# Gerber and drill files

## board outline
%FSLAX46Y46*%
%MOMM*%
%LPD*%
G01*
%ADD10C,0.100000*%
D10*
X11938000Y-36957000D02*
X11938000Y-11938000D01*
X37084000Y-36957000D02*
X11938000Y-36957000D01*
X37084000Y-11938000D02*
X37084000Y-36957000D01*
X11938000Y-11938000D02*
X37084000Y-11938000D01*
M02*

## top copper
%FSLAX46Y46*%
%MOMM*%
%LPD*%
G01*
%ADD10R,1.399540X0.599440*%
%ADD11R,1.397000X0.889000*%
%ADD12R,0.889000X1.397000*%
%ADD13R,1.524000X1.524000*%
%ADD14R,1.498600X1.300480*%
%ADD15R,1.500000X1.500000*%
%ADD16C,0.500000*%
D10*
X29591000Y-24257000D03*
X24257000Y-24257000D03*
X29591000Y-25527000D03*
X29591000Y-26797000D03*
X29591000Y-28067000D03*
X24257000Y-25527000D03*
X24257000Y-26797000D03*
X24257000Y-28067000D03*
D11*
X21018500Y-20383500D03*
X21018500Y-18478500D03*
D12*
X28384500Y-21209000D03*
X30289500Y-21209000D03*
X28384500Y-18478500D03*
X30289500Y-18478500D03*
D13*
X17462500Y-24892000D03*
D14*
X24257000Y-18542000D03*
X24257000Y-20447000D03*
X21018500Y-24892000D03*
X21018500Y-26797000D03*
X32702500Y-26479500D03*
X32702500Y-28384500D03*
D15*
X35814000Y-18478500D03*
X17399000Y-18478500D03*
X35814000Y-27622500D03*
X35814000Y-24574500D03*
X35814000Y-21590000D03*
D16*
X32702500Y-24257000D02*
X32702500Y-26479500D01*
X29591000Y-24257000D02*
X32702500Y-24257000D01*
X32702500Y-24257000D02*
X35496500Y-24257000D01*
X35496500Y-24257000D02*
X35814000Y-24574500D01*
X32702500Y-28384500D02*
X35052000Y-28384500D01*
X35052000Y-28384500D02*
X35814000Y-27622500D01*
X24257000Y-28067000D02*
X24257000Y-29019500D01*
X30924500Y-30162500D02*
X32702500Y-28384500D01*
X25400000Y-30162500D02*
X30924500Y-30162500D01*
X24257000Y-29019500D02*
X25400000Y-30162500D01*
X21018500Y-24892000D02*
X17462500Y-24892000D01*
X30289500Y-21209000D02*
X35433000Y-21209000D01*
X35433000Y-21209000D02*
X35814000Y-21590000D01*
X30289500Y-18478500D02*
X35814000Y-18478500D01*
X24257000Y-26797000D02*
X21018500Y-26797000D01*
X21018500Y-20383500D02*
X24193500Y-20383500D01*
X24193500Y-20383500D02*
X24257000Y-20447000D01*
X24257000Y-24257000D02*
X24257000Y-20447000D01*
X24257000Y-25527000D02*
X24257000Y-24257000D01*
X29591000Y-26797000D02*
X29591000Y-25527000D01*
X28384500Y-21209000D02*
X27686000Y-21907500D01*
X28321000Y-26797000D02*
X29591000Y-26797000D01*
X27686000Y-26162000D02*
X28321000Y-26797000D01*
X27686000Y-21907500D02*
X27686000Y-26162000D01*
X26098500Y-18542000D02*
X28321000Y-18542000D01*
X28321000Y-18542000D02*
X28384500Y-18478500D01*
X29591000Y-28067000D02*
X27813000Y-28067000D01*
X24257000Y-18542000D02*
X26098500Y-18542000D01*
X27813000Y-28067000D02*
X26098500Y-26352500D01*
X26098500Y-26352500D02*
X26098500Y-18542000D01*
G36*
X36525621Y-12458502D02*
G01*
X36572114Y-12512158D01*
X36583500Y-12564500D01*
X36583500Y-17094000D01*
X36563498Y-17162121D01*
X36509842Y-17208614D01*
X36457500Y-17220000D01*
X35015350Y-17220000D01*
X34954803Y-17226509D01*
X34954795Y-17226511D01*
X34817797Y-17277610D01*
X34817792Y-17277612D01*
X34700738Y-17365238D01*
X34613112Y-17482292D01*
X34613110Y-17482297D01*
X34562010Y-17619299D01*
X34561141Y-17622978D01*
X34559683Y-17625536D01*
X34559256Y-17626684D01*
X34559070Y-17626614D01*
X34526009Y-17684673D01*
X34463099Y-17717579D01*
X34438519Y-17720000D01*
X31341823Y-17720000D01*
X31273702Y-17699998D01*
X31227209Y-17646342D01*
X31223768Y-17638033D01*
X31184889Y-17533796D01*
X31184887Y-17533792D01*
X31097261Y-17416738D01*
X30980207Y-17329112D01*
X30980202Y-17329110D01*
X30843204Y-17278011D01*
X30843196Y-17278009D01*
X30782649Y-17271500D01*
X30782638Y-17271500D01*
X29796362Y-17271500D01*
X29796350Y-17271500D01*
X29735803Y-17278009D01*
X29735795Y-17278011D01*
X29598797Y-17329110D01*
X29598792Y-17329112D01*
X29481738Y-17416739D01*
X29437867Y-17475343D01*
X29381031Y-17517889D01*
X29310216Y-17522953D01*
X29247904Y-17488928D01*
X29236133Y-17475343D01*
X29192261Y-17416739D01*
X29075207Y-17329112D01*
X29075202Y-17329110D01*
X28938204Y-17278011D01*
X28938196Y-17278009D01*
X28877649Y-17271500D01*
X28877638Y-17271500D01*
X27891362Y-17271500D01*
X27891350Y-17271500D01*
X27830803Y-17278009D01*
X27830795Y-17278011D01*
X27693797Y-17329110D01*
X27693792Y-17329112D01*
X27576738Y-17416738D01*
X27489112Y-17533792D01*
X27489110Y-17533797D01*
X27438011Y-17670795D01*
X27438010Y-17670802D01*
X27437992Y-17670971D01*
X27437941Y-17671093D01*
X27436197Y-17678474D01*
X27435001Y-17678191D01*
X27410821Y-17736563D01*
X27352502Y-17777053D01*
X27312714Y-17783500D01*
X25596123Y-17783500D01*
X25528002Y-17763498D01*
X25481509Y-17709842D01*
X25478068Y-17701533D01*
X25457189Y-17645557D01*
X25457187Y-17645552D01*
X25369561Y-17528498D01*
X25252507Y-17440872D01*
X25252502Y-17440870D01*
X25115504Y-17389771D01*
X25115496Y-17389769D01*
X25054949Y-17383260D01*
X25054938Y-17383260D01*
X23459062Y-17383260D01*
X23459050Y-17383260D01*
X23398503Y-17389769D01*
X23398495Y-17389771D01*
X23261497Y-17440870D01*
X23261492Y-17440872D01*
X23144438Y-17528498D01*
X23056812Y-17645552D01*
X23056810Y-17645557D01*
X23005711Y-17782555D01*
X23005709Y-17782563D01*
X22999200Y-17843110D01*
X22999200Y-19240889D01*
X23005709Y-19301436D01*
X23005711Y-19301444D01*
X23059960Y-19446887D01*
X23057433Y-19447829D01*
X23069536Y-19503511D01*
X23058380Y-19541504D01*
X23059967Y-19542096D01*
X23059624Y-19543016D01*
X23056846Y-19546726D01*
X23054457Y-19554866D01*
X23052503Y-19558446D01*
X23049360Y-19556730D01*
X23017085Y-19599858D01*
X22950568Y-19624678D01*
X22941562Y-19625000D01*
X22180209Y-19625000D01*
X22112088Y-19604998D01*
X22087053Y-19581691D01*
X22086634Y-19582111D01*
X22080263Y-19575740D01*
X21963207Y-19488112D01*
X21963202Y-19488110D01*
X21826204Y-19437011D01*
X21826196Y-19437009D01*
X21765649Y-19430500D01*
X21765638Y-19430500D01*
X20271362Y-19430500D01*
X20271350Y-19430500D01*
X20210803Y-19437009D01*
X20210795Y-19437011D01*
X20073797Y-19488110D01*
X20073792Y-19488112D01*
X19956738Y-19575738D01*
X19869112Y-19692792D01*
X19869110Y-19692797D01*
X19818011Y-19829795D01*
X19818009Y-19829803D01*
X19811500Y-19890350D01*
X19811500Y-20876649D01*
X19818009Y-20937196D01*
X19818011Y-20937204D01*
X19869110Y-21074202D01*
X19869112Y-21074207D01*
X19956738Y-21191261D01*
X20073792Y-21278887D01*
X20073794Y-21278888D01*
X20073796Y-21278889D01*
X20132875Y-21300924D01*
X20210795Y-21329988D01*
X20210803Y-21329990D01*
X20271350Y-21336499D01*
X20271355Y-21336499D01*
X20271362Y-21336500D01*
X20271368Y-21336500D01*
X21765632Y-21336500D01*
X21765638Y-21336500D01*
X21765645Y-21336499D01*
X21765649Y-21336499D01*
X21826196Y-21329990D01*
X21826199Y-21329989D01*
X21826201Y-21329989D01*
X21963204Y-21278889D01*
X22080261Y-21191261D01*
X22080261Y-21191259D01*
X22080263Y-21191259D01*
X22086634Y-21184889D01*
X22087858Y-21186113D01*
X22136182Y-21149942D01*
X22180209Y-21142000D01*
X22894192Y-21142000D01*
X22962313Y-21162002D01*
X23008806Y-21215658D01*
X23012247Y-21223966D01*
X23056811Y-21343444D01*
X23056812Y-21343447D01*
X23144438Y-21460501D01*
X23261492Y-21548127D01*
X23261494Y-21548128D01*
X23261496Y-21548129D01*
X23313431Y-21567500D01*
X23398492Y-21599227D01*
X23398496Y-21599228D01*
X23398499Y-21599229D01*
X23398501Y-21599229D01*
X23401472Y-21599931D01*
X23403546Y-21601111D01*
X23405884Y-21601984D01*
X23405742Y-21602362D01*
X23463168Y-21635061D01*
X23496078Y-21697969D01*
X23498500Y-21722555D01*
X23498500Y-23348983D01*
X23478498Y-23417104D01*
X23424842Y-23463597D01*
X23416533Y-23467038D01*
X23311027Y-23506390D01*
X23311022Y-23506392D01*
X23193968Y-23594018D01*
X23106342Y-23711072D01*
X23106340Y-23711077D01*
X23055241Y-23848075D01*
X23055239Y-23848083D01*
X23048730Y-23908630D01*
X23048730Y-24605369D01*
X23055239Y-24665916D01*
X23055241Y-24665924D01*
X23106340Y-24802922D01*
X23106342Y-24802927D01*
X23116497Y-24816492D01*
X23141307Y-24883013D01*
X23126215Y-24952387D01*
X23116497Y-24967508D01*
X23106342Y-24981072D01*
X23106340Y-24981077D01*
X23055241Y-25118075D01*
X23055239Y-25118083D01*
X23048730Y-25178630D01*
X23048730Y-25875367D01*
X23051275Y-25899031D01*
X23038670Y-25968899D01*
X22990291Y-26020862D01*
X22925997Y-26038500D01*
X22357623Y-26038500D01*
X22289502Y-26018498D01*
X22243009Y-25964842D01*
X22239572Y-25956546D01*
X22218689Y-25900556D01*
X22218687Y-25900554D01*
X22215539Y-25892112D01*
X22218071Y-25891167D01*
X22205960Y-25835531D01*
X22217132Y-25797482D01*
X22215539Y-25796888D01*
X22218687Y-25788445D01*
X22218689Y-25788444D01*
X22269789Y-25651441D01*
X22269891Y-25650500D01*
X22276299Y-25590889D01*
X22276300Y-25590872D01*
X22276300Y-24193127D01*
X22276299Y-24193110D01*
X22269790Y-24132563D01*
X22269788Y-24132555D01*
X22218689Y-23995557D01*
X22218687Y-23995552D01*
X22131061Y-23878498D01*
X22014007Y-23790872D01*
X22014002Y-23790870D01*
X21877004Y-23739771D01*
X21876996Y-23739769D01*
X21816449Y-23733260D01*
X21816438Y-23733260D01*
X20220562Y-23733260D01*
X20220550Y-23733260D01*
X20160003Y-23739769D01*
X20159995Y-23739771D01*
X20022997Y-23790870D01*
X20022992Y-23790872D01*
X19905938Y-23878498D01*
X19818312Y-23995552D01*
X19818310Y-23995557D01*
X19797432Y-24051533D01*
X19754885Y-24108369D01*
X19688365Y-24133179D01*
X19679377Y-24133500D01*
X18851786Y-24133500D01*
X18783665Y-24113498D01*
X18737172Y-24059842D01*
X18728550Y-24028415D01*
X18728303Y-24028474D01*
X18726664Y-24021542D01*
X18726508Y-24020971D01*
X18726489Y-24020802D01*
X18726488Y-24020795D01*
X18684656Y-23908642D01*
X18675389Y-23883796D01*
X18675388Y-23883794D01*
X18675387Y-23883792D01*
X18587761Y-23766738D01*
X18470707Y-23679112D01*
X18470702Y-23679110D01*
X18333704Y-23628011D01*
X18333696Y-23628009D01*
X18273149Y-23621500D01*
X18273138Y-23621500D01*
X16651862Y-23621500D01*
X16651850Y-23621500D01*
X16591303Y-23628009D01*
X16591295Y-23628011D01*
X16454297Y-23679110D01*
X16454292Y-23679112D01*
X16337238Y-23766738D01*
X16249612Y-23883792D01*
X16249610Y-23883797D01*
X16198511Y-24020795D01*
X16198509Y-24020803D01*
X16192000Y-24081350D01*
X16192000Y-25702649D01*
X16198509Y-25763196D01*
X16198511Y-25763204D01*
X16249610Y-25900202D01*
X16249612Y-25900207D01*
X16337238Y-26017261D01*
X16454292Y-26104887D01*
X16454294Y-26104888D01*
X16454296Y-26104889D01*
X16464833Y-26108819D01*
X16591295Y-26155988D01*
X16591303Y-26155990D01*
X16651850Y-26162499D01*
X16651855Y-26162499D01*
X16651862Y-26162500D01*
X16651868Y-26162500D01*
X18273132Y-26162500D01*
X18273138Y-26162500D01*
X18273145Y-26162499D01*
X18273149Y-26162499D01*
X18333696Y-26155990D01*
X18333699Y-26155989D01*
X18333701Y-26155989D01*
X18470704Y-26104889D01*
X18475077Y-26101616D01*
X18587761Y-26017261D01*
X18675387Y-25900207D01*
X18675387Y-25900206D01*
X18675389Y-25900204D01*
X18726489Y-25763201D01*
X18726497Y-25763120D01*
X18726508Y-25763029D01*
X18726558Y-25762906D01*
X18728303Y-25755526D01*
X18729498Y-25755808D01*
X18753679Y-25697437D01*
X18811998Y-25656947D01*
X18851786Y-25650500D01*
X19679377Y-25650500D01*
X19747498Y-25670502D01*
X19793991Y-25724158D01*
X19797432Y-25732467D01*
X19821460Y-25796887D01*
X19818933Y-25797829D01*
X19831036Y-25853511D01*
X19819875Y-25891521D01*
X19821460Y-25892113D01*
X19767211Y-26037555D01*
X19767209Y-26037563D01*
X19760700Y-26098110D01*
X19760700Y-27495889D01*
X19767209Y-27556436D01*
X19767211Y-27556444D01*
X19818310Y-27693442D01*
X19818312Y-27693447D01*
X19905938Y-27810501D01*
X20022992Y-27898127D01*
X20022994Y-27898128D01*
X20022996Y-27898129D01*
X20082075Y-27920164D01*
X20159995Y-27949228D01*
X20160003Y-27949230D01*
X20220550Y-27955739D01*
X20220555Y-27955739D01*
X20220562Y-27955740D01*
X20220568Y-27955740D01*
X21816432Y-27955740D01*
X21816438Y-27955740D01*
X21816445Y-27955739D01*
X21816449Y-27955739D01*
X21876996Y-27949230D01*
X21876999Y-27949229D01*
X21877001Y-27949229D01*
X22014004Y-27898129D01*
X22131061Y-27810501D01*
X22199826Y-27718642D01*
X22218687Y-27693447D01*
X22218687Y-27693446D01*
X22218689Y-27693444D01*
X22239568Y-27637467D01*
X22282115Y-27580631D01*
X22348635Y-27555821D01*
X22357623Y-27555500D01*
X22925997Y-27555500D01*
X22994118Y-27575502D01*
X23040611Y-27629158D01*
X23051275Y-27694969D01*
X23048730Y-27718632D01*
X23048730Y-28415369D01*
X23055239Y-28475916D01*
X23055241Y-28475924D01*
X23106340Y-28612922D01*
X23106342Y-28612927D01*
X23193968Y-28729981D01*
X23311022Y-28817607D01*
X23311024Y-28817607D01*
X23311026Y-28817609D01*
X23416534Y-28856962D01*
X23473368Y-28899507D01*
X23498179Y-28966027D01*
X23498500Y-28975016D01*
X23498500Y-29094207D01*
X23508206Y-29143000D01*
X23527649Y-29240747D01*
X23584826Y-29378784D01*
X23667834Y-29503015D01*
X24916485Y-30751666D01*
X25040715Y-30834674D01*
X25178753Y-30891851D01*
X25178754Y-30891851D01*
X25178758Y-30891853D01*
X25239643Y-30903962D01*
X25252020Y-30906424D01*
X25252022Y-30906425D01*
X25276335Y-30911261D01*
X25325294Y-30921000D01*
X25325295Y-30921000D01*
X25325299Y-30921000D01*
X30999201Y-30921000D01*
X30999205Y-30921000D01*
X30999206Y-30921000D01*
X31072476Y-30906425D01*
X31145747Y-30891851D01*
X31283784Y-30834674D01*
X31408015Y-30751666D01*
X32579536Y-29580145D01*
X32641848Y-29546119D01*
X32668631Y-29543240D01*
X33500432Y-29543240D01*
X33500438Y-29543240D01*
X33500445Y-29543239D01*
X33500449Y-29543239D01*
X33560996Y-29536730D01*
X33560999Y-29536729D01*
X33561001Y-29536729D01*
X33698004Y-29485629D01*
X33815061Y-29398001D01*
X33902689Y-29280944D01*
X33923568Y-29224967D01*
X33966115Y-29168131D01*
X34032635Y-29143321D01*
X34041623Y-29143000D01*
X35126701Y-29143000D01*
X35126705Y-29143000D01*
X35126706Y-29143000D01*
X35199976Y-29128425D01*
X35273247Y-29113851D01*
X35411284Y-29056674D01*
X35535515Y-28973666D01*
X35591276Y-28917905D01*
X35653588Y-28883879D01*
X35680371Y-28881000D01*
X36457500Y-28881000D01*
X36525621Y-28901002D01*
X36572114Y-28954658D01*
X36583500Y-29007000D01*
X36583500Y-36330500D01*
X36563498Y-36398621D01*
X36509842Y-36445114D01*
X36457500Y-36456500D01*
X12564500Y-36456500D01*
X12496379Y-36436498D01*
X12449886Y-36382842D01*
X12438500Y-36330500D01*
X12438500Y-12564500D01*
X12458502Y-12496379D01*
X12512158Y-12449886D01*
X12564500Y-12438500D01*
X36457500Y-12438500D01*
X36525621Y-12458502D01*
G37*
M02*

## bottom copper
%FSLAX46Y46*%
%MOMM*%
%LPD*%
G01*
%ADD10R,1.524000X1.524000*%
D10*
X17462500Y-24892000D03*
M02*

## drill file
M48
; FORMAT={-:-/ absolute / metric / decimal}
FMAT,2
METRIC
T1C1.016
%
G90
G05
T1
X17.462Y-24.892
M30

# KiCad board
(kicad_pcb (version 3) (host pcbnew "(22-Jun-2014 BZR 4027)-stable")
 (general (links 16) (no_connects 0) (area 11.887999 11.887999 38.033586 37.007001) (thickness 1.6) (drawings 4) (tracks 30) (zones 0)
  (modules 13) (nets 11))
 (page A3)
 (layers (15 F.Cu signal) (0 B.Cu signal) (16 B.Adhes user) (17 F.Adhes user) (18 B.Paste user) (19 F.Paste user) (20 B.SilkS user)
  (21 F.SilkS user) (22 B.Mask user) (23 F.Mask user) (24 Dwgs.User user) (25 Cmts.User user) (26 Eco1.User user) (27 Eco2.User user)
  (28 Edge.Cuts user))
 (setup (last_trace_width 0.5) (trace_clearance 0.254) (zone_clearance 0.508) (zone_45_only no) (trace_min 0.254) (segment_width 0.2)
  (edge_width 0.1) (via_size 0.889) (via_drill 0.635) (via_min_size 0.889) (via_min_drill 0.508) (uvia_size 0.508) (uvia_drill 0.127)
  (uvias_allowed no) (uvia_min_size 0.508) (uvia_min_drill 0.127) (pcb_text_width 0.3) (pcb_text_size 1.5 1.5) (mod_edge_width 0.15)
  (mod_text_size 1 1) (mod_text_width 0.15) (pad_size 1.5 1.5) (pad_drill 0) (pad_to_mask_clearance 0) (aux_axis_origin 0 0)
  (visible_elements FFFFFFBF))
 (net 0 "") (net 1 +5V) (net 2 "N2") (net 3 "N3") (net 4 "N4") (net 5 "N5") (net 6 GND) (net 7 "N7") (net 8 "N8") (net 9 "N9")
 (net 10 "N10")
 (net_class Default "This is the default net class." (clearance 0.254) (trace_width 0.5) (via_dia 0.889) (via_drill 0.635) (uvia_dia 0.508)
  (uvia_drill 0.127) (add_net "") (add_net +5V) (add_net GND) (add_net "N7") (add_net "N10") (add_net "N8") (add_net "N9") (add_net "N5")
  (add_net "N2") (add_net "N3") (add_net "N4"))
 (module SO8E (layer F.Cu) (at 26.924 26.162 270)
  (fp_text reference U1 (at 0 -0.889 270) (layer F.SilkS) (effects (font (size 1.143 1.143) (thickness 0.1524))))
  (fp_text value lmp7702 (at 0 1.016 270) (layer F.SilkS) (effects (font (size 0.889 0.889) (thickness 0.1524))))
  (pad 8 smd rect (at -1.905 -2.667 270) (size 0.59944 1.39954) (layers F.Cu F.Paste F.Mask) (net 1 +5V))
  (pad 1 smd rect (at -1.905 2.667 270) (size 0.59944 1.39954) (layers F.Cu F.Paste F.Mask) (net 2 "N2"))
  (pad 7 smd rect (at -0.635 -2.667 270) (size 0.59944 1.39954) (layers F.Cu F.Paste F.Mask) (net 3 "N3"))
  (pad 6 smd rect (at 0.635 -2.667 270) (size 0.59944 1.39954) (layers F.Cu F.Paste F.Mask) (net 3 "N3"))
  (pad 5 smd rect (at 1.905 -2.667 270) (size 0.59944 1.39954) (layers F.Cu F.Paste F.Mask) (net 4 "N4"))
  (pad 2 smd rect (at -0.635 2.667 270) (size 0.59944 1.39954) (layers F.Cu F.Paste F.Mask) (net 2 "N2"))
  (pad 3 smd rect (at 0.635 2.667 270) (size 0.59944 1.39954) (layers F.Cu F.Paste F.Mask) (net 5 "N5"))
  (pad 4 smd rect (at 1.905 2.667 270) (size 0.59944 1.39954) (layers F.Cu F.Paste F.Mask) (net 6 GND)))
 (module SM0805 (layer F.Cu) (at 21.0185 19.431 90)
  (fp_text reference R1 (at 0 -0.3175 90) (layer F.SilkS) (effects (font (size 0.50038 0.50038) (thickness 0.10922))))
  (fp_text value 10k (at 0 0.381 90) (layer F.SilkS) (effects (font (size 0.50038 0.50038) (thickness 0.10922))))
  (pad 1 smd rect (at -0.9525 0 90) (size 0.889 1.397) (layers F.Cu F.Paste F.Mask) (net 2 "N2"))
  (pad 2 smd rect (at 0.9525 0 90) (size 0.889 1.397) (layers F.Cu F.Paste F.Mask) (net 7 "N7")))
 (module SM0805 (layer F.Cu) (at 29.337 21.209)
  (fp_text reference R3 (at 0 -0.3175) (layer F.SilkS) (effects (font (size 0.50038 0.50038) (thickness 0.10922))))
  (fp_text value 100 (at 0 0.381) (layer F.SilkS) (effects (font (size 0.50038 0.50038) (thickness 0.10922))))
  (pad 1 smd rect (at -0.9525 0) (size 0.889 1.397) (layers F.Cu F.Paste F.Mask) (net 3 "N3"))
  (pad 2 smd rect (at 0.9525 0) (size 0.889 1.397) (layers F.Cu F.Paste F.Mask) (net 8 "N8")))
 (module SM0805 (layer F.Cu) (at 29.337 18.4785)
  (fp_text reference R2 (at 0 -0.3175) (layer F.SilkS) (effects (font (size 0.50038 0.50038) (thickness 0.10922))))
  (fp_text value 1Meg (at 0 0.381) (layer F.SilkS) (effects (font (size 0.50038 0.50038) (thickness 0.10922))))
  (pad 1 smd rect (at -0.9525 0) (size 0.889 1.397) (layers F.Cu F.Paste F.Mask) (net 4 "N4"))
  (pad 2 smd rect (at 0.9525 0) (size 0.889 1.397) (layers F.Cu F.Paste F.Mask) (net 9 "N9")))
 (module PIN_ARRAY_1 (layer F.Cu) (at 17.4625 24.892)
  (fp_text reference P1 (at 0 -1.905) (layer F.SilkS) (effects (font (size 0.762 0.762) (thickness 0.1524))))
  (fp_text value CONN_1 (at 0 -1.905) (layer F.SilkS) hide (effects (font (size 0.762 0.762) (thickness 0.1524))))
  (pad 1 thru_hole rect (at 0 0) (size 1.524 1.524) (drill 1.016) (layers *.Cu *.Mask F.SilkS) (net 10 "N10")))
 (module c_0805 (layer F.Cu) (at 24.257 19.4945 90)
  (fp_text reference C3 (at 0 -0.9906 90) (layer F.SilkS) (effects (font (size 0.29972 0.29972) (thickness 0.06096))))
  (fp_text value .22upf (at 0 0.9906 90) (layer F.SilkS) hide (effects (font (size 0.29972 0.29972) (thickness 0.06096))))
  (pad 1 smd rect (at 0.9525 0 90) (size 1.30048 1.4986) (layers F.Cu F.Paste F.Mask) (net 4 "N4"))
  (pad 2 smd rect (at -0.9525 0 90) (size 1.30048 1.4986) (layers F.Cu F.Paste F.Mask) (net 2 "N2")))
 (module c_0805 (layer F.Cu) (at 21.0185 25.8445 90)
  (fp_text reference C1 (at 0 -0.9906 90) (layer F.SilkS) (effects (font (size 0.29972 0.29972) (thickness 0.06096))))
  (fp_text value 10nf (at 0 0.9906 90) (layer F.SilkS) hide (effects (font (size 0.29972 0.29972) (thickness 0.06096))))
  (pad 1 smd rect (at 0.9525 0 90) (size 1.30048 1.4986) (layers F.Cu F.Paste F.Mask) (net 10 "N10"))
  (pad 2 smd rect (at -0.9525 0 90) (size 1.30048 1.4986) (layers F.Cu F.Paste F.Mask) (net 5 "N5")))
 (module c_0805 (layer F.Cu) (at 32.7025 27.432 90)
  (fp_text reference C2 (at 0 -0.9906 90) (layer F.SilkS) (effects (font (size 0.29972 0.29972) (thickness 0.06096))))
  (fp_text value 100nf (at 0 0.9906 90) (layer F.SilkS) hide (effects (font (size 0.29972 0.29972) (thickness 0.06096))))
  (pad 1 smd rect (at 0.9525 0 90) (size 1.30048 1.4986) (layers F.Cu F.Paste F.Mask) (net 1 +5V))
  (pad 2 smd rect (at -0.9525 0 90) (size 1.30048 1.4986) (layers F.Cu F.Paste F.Mask) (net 6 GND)))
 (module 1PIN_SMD (layer F.Cu) (at 35.814 18.4785)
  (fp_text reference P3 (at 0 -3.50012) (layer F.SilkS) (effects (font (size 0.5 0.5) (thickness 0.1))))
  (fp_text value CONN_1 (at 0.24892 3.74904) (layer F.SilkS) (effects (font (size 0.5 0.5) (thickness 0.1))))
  (pad 1 smd rect (at 0 0) (size 1.5 1.5) (layers F.Cu F.Paste F.SilkS F.Mask) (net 9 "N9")))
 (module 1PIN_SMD (layer F.Cu) (at 17.399 18.4785)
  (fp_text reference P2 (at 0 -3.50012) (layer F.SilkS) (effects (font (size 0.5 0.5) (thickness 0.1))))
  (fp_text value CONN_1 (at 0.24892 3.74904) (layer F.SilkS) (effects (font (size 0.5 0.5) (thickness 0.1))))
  (pad 1 smd rect (at 0 0) (size 1.5 1.5) (layers F.Cu F.Paste F.SilkS F.Mask) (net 7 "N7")))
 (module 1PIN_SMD (layer F.Cu) (at 35.814 27.6225)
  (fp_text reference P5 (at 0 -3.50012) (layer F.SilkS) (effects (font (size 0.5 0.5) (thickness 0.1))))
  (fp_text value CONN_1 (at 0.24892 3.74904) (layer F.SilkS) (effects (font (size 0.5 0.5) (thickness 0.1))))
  (pad 1 smd rect (at 0 0) (size 1.5 1.5) (layers F.Cu F.Paste F.SilkS F.Mask) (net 6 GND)))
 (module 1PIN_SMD (layer F.Cu) (at 35.814 24.5745)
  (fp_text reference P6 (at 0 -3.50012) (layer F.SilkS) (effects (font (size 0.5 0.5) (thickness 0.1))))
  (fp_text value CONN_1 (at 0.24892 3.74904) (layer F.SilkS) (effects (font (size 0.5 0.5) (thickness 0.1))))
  (pad 1 smd rect (at 0 0) (size 1.5 1.5) (layers F.Cu F.Paste F.SilkS F.Mask) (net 1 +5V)))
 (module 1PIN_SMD (layer F.Cu) (at 35.814 21.59)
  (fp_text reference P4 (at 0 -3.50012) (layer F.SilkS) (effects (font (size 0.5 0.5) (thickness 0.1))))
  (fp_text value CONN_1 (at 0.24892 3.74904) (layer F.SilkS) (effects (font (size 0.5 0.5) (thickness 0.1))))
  (pad 1 smd rect (at 0 0) (size 1.5 1.5) (layers F.Cu F.Paste F.SilkS F.Mask) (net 8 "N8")))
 (gr_line (start 11.938 36.957) (end 11.938 11.938) (angle 90) (layer Edge.Cuts) (width 0.1))
 (gr_line (start 37.084 36.957) (end 11.938 36.957) (angle 90) (layer Edge.Cuts) (width 0.1))
 (gr_line (start 37.084 11.938) (end 37.084 36.957) (angle 90) (layer Edge.Cuts) (width 0.1))
 (gr_line (start 11.938 11.938) (end 37.084 11.938) (angle 90) (layer Edge.Cuts) (width 0.1))
 (segment (start 32.7025 24.257) (end 32.7025 26.4795) (width 0.5) (layer F.Cu) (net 1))
 (segment (start 29.591 24.257) (end 32.7025 24.257) (width 0.5) (layer F.Cu) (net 1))
 (segment (start 32.7025 24.257) (end 35.4965 24.257) (width 0.5) (layer F.Cu) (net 1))
 (segment (start 35.4965 24.257) (end 35.814 24.5745) (width 0.5) (layer F.Cu) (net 1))
 (segment (start 32.7025 28.3845) (end 35.052 28.3845) (width 0.5) (layer F.Cu) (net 6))
 (segment (start 35.052 28.3845) (end 35.814 27.6225) (width 0.5) (layer F.Cu) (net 6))
 (segment (start 24.257 28.067) (end 24.257 29.0195) (width 0.5) (layer F.Cu) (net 6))
 (segment (start 30.9245 30.1625) (end 32.7025 28.3845) (width 0.5) (layer F.Cu) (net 6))
 (segment (start 25.4 30.1625) (end 30.9245 30.1625) (width 0.5) (layer F.Cu) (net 6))
 (segment (start 24.257 29.0195) (end 25.4 30.1625) (width 0.5) (layer F.Cu) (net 6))
 (segment (start 21.0185 24.892) (end 17.4625 24.892) (width 0.5) (layer F.Cu) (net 10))
 (segment (start 30.2895 21.209) (end 35.433 21.209) (width 0.5) (layer F.Cu) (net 8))
 (segment (start 35.433 21.209) (end 35.814 21.59) (width 0.5) (layer F.Cu) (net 8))
 (segment (start 30.2895 18.4785) (end 35.814 18.4785) (width 0.5) (layer F.Cu) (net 9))
 (segment (start 24.257 26.797) (end 21.0185 26.797) (width 0.5) (layer F.Cu) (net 5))
 (segment (start 21.0185 20.3835) (end 24.1935 20.3835) (width 0.5) (layer F.Cu) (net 2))
 (segment (start 24.1935 20.3835) (end 24.257 20.447) (width 0.5) (layer F.Cu) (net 2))
 (segment (start 24.257 24.257) (end 24.257 20.447) (width 0.5) (layer F.Cu) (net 2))
 (segment (start 24.257 25.527) (end 24.257 24.257) (width 0.5) (layer F.Cu) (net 2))
 (segment (start 29.591 26.797) (end 29.591 25.527) (width 0.5) (layer F.Cu) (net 3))
 (segment (start 28.3845 21.209) (end 27.686 21.9075) (width 0.5) (layer F.Cu) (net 3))
 (segment (start 28.321 26.797) (end 29.591 26.797) (width 0.5) (layer F.Cu) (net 3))
 (segment (start 27.686 26.162) (end 28.321 26.797) (width 0.5) (layer F.Cu) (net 3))
 (segment (start 27.686 21.9075) (end 27.686 26.162) (width 0.5) (layer F.Cu) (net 3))
 (segment (start 26.0985 18.542) (end 28.321 18.542) (width 0.5) (layer F.Cu) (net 4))
 (segment (start 28.321 18.542) (end 28.3845 18.4785) (width 0.5) (layer F.Cu) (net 4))
 (segment (start 29.591 28.067) (end 27.813 28.067) (width 0.5) (layer F.Cu) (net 4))
 (segment (start 24.257 18.542) (end 26.0985 18.542) (width 0.5) (layer F.Cu) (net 4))
 (segment (start 27.813 28.067) (end 26.0985 26.3525) (width 0.5) (layer F.Cu) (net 4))
 (segment (start 26.0985 26.3525) (end 26.0985 18.542) (width 0.5) (layer F.Cu) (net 4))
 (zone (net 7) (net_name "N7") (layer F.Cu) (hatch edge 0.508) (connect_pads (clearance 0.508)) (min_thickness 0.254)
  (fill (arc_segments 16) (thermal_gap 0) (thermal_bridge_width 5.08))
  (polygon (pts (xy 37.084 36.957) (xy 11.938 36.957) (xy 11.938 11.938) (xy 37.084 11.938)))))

